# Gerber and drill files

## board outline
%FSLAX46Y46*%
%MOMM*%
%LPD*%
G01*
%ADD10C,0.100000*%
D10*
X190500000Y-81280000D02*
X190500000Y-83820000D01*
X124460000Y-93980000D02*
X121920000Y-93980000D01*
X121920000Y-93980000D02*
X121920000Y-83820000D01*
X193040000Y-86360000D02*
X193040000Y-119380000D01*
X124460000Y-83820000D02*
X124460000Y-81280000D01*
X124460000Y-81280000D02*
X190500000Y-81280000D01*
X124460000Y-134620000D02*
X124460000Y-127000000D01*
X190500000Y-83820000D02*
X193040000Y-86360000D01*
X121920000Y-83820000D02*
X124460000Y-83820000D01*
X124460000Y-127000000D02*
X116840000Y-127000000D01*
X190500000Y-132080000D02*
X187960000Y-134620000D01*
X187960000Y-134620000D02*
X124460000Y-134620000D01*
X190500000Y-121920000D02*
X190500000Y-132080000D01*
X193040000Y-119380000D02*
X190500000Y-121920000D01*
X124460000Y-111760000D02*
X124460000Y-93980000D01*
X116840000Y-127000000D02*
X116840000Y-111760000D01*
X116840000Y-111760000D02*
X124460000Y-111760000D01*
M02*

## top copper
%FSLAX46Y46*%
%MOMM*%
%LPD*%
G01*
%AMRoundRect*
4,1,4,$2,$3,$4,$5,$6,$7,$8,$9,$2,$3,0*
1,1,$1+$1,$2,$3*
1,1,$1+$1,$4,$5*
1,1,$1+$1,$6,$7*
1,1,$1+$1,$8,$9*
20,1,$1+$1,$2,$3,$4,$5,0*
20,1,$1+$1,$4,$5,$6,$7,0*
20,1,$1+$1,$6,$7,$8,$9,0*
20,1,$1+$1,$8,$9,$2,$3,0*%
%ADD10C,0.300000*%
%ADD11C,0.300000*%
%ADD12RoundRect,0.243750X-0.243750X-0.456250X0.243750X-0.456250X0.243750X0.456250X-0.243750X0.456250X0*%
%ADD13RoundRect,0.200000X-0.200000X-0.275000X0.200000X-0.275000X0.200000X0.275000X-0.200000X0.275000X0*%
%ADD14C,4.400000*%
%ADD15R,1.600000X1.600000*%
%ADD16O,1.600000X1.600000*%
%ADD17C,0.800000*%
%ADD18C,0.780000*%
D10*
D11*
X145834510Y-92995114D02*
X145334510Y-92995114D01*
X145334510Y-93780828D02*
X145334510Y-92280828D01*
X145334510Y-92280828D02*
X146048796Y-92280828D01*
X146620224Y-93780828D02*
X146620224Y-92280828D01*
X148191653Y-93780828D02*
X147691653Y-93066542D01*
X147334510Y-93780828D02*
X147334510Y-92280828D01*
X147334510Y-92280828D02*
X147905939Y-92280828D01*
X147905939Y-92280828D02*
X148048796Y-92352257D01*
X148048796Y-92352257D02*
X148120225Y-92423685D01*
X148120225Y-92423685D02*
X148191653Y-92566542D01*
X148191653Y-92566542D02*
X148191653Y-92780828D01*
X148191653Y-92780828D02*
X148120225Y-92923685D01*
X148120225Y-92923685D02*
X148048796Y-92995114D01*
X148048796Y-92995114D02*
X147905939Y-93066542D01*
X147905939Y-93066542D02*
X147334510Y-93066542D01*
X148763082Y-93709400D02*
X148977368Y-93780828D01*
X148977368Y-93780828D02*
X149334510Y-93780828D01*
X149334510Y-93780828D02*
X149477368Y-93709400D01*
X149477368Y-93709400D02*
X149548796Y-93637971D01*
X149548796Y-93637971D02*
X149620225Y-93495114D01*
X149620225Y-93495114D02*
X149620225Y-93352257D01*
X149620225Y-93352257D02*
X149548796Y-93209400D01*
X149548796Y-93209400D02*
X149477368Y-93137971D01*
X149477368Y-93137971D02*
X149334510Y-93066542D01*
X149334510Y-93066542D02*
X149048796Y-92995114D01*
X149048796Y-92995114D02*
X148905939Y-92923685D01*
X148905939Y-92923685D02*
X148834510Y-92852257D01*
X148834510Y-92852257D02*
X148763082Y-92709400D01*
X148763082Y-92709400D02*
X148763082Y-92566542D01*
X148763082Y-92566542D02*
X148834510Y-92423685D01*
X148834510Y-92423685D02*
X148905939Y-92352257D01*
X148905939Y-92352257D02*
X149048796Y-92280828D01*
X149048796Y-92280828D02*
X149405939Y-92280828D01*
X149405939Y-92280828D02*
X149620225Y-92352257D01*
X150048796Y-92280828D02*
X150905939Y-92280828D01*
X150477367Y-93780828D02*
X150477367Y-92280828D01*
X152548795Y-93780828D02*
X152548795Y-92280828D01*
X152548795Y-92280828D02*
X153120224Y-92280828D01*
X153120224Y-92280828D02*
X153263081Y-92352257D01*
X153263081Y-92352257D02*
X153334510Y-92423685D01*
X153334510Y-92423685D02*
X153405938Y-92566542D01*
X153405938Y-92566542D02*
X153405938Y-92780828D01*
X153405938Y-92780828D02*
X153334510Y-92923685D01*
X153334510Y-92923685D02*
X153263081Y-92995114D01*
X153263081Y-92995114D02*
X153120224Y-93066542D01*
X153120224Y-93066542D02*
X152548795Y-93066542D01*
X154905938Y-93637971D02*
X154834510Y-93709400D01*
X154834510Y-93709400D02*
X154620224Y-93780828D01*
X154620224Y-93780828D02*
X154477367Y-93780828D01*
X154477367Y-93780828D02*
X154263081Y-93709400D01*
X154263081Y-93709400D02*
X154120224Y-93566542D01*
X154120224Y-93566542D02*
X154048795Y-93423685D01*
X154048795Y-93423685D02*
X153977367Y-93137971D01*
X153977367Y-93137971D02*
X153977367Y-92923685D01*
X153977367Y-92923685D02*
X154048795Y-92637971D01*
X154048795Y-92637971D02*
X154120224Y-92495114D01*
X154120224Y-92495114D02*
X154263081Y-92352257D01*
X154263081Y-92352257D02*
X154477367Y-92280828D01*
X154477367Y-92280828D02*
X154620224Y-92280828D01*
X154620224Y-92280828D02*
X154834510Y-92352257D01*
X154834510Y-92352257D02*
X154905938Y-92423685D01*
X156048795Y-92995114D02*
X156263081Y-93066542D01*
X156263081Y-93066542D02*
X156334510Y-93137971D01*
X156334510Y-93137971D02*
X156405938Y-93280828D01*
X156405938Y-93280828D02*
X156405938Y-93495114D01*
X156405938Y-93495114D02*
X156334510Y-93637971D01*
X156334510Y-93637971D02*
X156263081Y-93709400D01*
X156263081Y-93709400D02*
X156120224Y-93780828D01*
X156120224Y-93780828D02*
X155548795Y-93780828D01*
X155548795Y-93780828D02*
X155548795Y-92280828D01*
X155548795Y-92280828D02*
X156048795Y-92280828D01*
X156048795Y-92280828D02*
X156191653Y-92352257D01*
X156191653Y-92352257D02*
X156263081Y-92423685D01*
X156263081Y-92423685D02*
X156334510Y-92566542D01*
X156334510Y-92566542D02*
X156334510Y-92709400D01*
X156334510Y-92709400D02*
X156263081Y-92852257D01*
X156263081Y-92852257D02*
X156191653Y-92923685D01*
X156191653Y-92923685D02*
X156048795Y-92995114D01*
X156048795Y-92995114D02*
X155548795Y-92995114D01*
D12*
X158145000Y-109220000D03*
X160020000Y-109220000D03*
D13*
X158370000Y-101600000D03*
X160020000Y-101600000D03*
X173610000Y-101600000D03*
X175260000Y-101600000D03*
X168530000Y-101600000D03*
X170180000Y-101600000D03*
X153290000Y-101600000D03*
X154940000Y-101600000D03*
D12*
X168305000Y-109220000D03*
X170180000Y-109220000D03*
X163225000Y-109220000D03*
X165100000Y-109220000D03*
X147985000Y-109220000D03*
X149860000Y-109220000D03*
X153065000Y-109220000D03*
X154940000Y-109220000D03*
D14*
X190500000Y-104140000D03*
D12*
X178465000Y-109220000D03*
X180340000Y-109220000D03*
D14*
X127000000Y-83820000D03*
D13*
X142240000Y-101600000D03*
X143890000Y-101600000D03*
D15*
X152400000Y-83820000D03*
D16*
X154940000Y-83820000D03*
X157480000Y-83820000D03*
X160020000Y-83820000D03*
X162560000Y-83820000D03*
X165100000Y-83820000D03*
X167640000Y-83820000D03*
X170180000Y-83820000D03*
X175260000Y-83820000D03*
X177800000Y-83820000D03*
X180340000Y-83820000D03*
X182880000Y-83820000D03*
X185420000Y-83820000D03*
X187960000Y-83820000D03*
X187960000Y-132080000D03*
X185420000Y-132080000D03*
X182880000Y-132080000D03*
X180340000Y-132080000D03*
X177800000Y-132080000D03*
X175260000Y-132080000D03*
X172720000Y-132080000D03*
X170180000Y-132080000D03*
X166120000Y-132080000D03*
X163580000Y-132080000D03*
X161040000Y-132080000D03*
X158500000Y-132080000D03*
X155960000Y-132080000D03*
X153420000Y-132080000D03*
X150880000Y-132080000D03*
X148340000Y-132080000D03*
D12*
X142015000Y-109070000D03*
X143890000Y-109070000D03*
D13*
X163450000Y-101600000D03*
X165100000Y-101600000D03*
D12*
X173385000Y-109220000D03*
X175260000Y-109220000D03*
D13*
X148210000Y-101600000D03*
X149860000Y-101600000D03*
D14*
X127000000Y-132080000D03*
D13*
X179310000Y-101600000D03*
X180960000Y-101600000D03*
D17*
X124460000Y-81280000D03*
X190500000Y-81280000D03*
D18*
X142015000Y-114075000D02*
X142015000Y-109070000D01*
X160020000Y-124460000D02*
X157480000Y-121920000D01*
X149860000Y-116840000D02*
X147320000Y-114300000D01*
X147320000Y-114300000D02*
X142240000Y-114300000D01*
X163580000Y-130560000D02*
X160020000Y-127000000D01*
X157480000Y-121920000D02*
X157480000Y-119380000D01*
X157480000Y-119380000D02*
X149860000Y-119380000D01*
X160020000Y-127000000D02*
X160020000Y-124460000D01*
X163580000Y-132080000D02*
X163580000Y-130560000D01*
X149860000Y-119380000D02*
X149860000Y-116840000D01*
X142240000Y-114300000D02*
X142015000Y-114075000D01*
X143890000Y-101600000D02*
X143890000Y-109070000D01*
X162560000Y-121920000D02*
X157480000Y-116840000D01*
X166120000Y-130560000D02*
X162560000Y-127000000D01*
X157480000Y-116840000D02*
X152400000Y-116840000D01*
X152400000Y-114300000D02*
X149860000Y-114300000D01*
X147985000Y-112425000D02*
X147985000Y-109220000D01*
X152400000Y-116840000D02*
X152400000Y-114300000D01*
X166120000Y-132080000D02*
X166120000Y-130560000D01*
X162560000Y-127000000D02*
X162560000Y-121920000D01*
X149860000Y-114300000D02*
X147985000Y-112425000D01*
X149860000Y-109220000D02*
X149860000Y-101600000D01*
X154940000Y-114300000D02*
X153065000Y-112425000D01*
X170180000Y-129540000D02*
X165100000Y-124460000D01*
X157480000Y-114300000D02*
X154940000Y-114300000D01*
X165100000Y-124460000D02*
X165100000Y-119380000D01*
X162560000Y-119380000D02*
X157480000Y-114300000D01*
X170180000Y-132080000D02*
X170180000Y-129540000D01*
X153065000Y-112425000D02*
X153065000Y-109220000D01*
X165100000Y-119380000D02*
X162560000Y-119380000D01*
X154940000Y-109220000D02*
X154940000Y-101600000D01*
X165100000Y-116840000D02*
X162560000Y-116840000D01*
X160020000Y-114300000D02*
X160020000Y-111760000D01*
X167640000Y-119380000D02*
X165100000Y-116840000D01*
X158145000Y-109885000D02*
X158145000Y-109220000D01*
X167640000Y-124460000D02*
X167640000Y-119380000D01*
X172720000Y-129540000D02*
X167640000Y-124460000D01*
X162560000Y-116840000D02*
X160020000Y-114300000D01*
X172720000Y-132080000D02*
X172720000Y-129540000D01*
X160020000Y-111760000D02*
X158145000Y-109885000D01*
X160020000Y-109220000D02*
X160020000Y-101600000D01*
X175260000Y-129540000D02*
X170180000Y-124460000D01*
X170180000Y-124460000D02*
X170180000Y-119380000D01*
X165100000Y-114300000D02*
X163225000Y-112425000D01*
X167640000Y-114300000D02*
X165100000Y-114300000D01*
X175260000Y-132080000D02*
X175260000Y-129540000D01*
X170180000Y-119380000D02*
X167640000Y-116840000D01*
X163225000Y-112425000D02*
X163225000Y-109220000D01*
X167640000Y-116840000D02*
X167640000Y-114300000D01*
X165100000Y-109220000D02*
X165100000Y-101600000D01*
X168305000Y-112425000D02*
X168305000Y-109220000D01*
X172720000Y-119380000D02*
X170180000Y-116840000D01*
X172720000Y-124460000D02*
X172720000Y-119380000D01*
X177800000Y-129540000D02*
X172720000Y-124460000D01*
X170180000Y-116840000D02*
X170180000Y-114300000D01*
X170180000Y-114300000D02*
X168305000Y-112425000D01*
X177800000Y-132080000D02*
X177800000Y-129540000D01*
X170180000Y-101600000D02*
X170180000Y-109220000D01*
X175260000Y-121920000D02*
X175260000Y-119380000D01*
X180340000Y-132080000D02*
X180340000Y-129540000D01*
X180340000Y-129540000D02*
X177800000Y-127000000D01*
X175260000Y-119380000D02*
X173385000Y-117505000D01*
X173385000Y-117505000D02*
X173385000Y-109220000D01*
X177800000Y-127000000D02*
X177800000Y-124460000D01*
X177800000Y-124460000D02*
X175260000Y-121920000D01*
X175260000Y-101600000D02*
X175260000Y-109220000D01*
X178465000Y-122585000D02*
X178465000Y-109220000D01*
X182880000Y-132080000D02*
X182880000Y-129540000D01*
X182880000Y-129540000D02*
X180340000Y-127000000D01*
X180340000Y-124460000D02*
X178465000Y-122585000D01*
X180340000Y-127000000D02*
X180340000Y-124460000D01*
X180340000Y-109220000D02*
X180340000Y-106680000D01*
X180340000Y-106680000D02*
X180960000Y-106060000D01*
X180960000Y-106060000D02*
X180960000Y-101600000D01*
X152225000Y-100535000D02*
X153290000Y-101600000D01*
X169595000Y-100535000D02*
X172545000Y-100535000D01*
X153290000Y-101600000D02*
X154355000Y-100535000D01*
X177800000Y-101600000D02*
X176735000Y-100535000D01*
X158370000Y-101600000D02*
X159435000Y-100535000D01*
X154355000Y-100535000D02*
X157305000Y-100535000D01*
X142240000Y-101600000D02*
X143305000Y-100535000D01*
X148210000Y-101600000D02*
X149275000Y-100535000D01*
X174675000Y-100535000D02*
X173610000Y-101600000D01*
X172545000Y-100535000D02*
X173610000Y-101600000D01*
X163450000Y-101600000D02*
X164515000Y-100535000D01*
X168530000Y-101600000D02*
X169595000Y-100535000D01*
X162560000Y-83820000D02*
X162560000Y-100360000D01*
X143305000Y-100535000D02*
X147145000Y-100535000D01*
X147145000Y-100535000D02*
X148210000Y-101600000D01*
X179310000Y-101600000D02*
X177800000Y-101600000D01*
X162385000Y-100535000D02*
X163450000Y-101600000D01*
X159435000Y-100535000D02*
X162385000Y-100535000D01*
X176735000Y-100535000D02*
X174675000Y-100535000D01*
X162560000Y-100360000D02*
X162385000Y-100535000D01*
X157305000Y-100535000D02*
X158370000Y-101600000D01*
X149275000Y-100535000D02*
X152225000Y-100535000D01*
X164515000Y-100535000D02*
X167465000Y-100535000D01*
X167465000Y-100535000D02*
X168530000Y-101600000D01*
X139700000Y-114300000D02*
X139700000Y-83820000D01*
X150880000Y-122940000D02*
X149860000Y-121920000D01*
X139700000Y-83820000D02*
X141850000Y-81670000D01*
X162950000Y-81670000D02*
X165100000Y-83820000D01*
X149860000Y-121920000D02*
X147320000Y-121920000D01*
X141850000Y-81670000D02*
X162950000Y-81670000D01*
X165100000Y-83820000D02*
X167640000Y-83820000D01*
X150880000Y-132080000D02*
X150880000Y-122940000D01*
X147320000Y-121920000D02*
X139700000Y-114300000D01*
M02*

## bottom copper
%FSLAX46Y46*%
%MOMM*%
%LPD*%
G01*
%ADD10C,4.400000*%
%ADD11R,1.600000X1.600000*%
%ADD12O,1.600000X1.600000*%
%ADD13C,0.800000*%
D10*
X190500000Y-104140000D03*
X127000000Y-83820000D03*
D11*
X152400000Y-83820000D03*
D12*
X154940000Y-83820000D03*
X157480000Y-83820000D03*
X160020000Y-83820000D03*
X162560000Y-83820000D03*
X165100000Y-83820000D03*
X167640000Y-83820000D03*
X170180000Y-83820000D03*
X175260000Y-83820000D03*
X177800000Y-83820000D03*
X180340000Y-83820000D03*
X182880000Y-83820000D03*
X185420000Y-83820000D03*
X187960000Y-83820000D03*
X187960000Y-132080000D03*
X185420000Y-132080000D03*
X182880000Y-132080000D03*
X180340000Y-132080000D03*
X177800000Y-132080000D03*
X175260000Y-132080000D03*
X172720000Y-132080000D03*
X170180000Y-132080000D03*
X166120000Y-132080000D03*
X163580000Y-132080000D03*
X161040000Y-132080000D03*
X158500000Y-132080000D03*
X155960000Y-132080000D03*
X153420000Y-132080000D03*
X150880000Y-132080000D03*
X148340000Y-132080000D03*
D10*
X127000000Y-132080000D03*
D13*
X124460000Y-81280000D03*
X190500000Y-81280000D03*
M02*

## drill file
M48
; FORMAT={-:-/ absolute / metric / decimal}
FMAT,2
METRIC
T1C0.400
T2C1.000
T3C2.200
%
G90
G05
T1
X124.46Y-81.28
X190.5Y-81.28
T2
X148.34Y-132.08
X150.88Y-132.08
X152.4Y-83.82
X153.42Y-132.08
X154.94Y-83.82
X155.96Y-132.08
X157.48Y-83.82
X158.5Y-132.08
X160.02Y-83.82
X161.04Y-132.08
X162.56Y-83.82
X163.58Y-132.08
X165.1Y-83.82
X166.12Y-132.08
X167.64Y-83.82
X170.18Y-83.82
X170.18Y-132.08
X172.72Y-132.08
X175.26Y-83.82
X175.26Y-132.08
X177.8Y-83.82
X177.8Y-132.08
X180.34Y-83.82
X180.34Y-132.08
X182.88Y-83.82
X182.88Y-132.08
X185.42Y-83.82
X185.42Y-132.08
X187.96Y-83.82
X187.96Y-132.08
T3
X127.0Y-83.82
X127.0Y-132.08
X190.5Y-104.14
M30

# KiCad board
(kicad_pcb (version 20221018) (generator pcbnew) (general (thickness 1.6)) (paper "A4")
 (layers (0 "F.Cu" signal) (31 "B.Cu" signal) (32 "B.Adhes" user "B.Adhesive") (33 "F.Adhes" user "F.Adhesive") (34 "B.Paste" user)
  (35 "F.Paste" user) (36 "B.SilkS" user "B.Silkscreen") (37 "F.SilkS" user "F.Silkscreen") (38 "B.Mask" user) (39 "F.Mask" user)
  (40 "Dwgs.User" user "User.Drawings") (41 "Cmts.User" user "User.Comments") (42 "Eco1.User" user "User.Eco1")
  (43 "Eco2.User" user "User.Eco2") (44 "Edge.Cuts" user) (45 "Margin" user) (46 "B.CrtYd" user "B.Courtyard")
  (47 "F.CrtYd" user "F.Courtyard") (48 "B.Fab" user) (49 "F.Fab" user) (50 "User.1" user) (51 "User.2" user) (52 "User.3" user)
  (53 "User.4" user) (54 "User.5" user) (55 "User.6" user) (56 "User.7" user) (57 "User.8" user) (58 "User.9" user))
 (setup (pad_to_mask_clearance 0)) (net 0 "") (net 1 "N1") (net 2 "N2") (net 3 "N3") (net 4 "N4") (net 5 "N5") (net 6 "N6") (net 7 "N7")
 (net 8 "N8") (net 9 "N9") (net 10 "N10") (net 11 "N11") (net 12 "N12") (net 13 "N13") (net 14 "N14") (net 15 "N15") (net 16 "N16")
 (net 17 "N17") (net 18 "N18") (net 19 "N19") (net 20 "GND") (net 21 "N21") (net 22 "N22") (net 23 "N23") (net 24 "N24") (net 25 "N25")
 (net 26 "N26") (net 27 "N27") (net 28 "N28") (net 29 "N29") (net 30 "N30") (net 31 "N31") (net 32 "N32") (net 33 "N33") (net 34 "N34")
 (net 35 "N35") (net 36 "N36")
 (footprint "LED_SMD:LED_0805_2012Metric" (layer "F.Cu") (at 159.0825 109.22)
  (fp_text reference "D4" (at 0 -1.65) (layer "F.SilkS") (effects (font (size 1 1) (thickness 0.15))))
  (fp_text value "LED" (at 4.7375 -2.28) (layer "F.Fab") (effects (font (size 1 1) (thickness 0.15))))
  (pad "1" smd roundrect (at -0.9375 0) (size 0.975 1.4) (layers "F.Cu" "F.Paste" "F.Mask") (roundrect_rratio 0.25) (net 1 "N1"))
  (pad "2" smd roundrect (at 0.9375 0) (size 0.975 1.4) (layers "F.Cu" "F.Paste" "F.Mask") (roundrect_rratio 0.25) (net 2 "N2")))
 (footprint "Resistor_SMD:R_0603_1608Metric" (layer "F.Cu") (at 159.195 101.6)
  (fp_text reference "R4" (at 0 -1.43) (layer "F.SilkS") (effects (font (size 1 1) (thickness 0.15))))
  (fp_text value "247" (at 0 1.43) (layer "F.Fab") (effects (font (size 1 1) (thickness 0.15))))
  (pad "1" smd roundrect (at -0.825 0) (size 0.8 0.95) (layers "F.Cu" "F.Paste" "F.Mask") (roundrect_rratio 0.25) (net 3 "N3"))
  (pad "2" smd roundrect (at 0.825 0) (size 0.8 0.95) (layers "F.Cu" "F.Paste" "F.Mask") (roundrect_rratio 0.25) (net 2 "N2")))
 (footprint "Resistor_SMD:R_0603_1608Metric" (layer "F.Cu") (at 174.435 101.6)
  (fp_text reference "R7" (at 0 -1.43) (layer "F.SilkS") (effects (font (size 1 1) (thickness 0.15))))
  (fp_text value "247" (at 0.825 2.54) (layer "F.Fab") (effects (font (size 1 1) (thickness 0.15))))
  (pad "1" smd roundrect (at -0.825 0) (size 0.8 0.95) (layers "F.Cu" "F.Paste" "F.Mask") (roundrect_rratio 0.25) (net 3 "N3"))
  (pad "2" smd roundrect (at 0.825 0) (size 0.8 0.95) (layers "F.Cu" "F.Paste" "F.Mask") (roundrect_rratio 0.25) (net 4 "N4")))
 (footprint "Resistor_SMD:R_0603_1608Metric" (layer "F.Cu") (at 169.355 101.6)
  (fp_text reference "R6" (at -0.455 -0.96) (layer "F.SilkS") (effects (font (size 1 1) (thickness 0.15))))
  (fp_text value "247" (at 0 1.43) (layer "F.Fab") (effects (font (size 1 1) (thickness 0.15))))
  (pad "1" smd roundrect (at -0.825 0) (size 0.8 0.95) (layers "F.Cu" "F.Paste" "F.Mask") (roundrect_rratio 0.25) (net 3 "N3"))
  (pad "2" smd roundrect (at 0.825 0) (size 0.8 0.95) (layers "F.Cu" "F.Paste" "F.Mask") (roundrect_rratio 0.25) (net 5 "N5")))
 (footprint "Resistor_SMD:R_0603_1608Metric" (layer "F.Cu") (at 154.115 101.6)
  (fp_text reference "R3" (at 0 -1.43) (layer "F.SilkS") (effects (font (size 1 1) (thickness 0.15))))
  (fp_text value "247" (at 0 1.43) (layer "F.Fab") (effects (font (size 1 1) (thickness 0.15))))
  (pad "1" smd roundrect (at -0.825 0) (size 0.8 0.95) (layers "F.Cu" "F.Paste" "F.Mask") (roundrect_rratio 0.25) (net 3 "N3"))
  (pad "2" smd roundrect (at 0.825 0) (size 0.8 0.95) (layers "F.Cu" "F.Paste" "F.Mask") (roundrect_rratio 0.25) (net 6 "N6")))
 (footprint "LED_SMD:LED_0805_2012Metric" (layer "F.Cu") (at 169.2425 109.22)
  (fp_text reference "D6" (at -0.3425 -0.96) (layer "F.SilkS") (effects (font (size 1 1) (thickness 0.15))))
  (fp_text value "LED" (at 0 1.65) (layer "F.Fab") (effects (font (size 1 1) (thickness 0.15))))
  (pad "1" smd roundrect (at -0.9375 0) (size 0.975 1.4) (layers "F.Cu" "F.Paste" "F.Mask") (roundrect_rratio 0.25) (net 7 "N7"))
  (pad "2" smd roundrect (at 0.9375 0) (size 0.975 1.4) (layers "F.Cu" "F.Paste" "F.Mask") (roundrect_rratio 0.25) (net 5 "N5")))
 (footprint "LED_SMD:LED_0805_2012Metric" (layer "F.Cu") (at 164.1625 109.22)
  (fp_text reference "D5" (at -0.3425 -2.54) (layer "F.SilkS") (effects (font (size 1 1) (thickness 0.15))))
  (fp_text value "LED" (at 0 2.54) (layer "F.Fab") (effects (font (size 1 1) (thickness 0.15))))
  (pad "1" smd roundrect (at -0.9375 0) (size 0.975 1.4) (layers "F.Cu" "F.Paste" "F.Mask") (roundrect_rratio 0.25) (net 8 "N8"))
  (pad "2" smd roundrect (at 0.9375 0) (size 0.975 1.4) (layers "F.Cu" "F.Paste" "F.Mask") (roundrect_rratio 0.25) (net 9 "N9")))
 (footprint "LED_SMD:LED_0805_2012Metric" (layer "F.Cu") (at 148.9225 109.22)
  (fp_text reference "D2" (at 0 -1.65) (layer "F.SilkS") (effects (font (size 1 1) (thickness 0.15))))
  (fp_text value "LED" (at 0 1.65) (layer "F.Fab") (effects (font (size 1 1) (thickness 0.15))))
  (pad "1" smd roundrect (at -0.9375 0) (size 0.975 1.4) (layers "F.Cu" "F.Paste" "F.Mask") (roundrect_rratio 0.25) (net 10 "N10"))
  (pad "2" smd roundrect (at 0.9375 0) (size 0.975 1.4) (layers "F.Cu" "F.Paste" "F.Mask") (roundrect_rratio 0.25) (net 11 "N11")))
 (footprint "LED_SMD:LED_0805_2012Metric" (layer "F.Cu") (at 154.0025 109.22)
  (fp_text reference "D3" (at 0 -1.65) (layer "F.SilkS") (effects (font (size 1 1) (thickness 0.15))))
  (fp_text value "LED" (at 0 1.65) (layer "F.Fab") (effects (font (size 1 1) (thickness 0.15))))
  (pad "1" smd roundrect (at -0.9375 0) (size 0.975 1.4) (layers "F.Cu" "F.Paste" "F.Mask") (roundrect_rratio 0.25) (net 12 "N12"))
  (pad "2" smd roundrect (at 0.9375 0) (size 0.975 1.4) (layers "F.Cu" "F.Paste" "F.Mask") (roundrect_rratio 0.25) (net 6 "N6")))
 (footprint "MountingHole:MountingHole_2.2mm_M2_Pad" (layer "F.Cu") (at 190.5 104.14)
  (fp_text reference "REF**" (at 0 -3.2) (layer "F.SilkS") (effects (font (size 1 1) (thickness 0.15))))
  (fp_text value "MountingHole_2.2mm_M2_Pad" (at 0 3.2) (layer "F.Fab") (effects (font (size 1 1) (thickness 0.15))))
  (pad "1" thru_hole circle (at 0 0) (size 4.4 4.4) (drill 2.2) (layers "*.Cu" "*.Mask")))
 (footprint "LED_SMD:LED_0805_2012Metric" (layer "F.Cu") (at 179.4025 109.22)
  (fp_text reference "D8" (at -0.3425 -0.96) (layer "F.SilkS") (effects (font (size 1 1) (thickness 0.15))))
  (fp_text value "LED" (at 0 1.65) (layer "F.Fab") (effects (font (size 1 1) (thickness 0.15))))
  (pad "1" smd roundrect (at -0.9375 0) (size 0.975 1.4) (layers "F.Cu" "F.Paste" "F.Mask") (roundrect_rratio 0.25) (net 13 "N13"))
  (pad "2" smd roundrect (at 0.9375 0) (size 0.975 1.4) (layers "F.Cu" "F.Paste" "F.Mask") (roundrect_rratio 0.25) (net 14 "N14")))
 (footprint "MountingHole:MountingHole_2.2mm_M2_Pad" (layer "F.Cu") (at 127 83.82)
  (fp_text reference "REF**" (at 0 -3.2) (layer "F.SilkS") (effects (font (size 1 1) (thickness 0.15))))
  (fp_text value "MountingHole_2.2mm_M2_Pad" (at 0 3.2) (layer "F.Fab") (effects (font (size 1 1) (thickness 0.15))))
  (pad "1" thru_hole circle (at 0 0) (size 4.4 4.4) (drill 2.2) (layers "*.Cu" "*.Mask")))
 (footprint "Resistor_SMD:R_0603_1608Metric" (layer "F.Cu") (at 143.065 101.6)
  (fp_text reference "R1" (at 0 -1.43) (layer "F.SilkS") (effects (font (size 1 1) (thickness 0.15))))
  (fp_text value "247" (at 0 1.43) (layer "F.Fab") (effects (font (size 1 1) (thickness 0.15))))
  (pad "1" smd roundrect (at -0.825 0) (size 0.8 0.95) (layers "F.Cu" "F.Paste" "F.Mask") (roundrect_rratio 0.25) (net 3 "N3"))
  (pad "2" smd roundrect (at 0.825 0) (size 0.8 0.95) (layers "F.Cu" "F.Paste" "F.Mask") (roundrect_rratio 0.25) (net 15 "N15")))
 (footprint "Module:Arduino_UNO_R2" (layer "F.Cu") (at 152.4 83.82)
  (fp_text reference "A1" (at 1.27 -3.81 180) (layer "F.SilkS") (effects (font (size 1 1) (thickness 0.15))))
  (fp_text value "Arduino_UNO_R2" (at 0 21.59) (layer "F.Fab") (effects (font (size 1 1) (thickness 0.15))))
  (pad "1" thru_hole rect (at 0 0 90) (size 1.6 1.6) (drill 1) (layers "*.Cu" "*.Mask") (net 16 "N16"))
  (pad "2" thru_hole oval (at 2.54 0 90) (size 1.6 1.6) (drill 1) (layers "*.Cu" "*.Mask") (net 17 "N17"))
  (pad "3" thru_hole oval (at 5.08 0 90) (size 1.6 1.6) (drill 1) (layers "*.Cu" "*.Mask") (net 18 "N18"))
  (pad "4" thru_hole oval (at 7.62 0 90) (size 1.6 1.6) (drill 1) (layers "*.Cu" "*.Mask") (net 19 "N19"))
  (pad "5" thru_hole oval (at 10.16 0 90) (size 1.6 1.6) (drill 1) (layers "*.Cu" "*.Mask") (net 3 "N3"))
  (pad "6" thru_hole oval (at 12.7 0 90) (size 1.6 1.6) (drill 1) (layers "*.Cu" "*.Mask") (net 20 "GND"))
  (pad "7" thru_hole oval (at 15.24 0 90) (size 1.6 1.6) (drill 1) (layers "*.Cu" "*.Mask") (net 20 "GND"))
  (pad "8" thru_hole oval (at 17.78 0 90) (size 1.6 1.6) (drill 1) (layers "*.Cu" "*.Mask") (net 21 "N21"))
  (pad "9" thru_hole oval (at 22.86 0 90) (size 1.6 1.6) (drill 1) (layers "*.Cu" "*.Mask") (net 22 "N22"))
  (pad "10" thru_hole oval (at 25.4 0 90) (size 1.6 1.6) (drill 1) (layers "*.Cu" "*.Mask") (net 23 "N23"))
  (pad "11" thru_hole oval (at 27.94 0 90) (size 1.6 1.6) (drill 1) (layers "*.Cu" "*.Mask") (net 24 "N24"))
  (pad "12" thru_hole oval (at 30.48 0 90) (size 1.6 1.6) (drill 1) (layers "*.Cu" "*.Mask") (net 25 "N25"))
  (pad "13" thru_hole oval (at 33.02 0 90) (size 1.6 1.6) (drill 1) (layers "*.Cu" "*.Mask") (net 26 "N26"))
  (pad "14" thru_hole oval (at 35.56 0 90) (size 1.6 1.6) (drill 1) (layers "*.Cu" "*.Mask") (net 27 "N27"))
  (pad "15" thru_hole oval (at 35.56 48.26 90) (size 1.6 1.6) (drill 1) (layers "*.Cu" "*.Mask") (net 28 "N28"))
  (pad "16" thru_hole oval (at 33.02 48.26 90) (size 1.6 1.6) (drill 1) (layers "*.Cu" "*.Mask") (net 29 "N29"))
  (pad "17" thru_hole oval (at 30.48 48.26 90) (size 1.6 1.6) (drill 1) (layers "*.Cu" "*.Mask") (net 13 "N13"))
  (pad "18" thru_hole oval (at 27.94 48.26 90) (size 1.6 1.6) (drill 1) (layers "*.Cu" "*.Mask") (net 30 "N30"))
  (pad "19" thru_hole oval (at 25.4 48.26 90) (size 1.6 1.6) (drill 1) (layers "*.Cu" "*.Mask") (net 7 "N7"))
  (pad "20" thru_hole oval (at 22.86 48.26 90) (size 1.6 1.6) (drill 1) (layers "*.Cu" "*.Mask") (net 8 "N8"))
  (pad "21" thru_hole oval (at 20.32 48.26 90) (size 1.6 1.6) (drill 1) (layers "*.Cu" "*.Mask") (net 1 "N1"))
  (pad "22" thru_hole oval (at 17.78 48.26 90) (size 1.6 1.6) (drill 1) (layers "*.Cu" "*.Mask") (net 12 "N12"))
  (pad "23" thru_hole oval (at 13.72 48.26 90) (size 1.6 1.6) (drill 1) (layers "*.Cu" "*.Mask") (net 10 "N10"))
  (pad "24" thru_hole oval (at 11.18 48.26 90) (size 1.6 1.6) (drill 1) (layers "*.Cu" "*.Mask") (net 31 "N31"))
  (pad "25" thru_hole oval (at 8.64 48.26 90) (size 1.6 1.6) (drill 1) (layers "*.Cu" "*.Mask") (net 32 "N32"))
  (pad "26" thru_hole oval (at 6.1 48.26 90) (size 1.6 1.6) (drill 1) (layers "*.Cu" "*.Mask") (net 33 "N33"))
  (pad "27" thru_hole oval (at 3.56 48.26 90) (size 1.6 1.6) (drill 1) (layers "*.Cu" "*.Mask") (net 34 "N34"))
  (pad "28" thru_hole oval (at 1.02 48.26 90) (size 1.6 1.6) (drill 1) (layers "*.Cu" "*.Mask") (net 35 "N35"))
  (pad "29" thru_hole oval (at -1.52 48.26 90) (size 1.6 1.6) (drill 1) (layers "*.Cu" "*.Mask") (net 20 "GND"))
  (pad "30" thru_hole oval (at -4.06 48.26 90) (size 1.6 1.6) (drill 1) (layers "*.Cu" "*.Mask") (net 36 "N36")))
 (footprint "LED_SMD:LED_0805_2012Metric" (layer "F.Cu") (at 142.9525 109.07)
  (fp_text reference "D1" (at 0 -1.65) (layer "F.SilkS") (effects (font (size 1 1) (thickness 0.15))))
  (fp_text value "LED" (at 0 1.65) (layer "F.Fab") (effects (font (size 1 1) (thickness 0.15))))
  (pad "1" smd roundrect (at -0.9375 0) (size 0.975 1.4) (layers "F.Cu" "F.Paste" "F.Mask") (roundrect_rratio 0.25) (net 31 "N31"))
  (pad "2" smd roundrect (at 0.9375 0) (size 0.975 1.4) (layers "F.Cu" "F.Paste" "F.Mask") (roundrect_rratio 0.25) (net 15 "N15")))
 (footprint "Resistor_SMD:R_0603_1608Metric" (layer "F.Cu") (at 164.275 101.6)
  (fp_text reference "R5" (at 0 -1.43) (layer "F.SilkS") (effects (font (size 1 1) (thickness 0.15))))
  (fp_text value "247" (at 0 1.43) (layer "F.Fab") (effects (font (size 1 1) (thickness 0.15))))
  (pad "1" smd roundrect (at -0.825 0) (size 0.8 0.95) (layers "F.Cu" "F.Paste" "F.Mask") (roundrect_rratio 0.25) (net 3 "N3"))
  (pad "2" smd roundrect (at 0.825 0) (size 0.8 0.95) (layers "F.Cu" "F.Paste" "F.Mask") (roundrect_rratio 0.25) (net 9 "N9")))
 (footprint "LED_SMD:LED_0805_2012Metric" (layer "F.Cu") (at 174.3225 109.22)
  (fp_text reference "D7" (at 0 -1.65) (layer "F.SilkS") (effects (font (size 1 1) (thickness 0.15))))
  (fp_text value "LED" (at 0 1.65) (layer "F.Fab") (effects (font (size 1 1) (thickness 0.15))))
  (pad "1" smd roundrect (at -0.9375 0) (size 0.975 1.4) (layers "F.Cu" "F.Paste" "F.Mask") (roundrect_rratio 0.25) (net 30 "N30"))
  (pad "2" smd roundrect (at 0.9375 0) (size 0.975 1.4) (layers "F.Cu" "F.Paste" "F.Mask") (roundrect_rratio 0.25) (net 4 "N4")))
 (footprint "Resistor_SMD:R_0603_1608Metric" (layer "F.Cu") (at 149.035 101.6)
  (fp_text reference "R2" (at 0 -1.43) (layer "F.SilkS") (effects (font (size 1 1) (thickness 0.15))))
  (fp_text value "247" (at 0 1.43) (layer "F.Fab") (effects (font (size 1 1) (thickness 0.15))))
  (pad "1" smd roundrect (at -0.825 0) (size 0.8 0.95) (layers "F.Cu" "F.Paste" "F.Mask") (roundrect_rratio 0.25) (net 3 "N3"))
  (pad "2" smd roundrect (at 0.825 0) (size 0.8 0.95) (layers "F.Cu" "F.Paste" "F.Mask") (roundrect_rratio 0.25) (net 11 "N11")))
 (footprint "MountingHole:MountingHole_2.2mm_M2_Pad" (layer "F.Cu") (at 127 132.08)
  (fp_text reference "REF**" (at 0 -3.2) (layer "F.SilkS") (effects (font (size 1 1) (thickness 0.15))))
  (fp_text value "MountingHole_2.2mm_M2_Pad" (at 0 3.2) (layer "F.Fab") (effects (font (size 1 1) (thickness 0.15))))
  (pad "1" thru_hole circle (at 0 0) (size 4.4 4.4) (drill 2.2) (layers "*.Cu" "*.Mask")))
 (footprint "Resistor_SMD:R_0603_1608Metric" (layer "F.Cu") (at 180.135 101.6)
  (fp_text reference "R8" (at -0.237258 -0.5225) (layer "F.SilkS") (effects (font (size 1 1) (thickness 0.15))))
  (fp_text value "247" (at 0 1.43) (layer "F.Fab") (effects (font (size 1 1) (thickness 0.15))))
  (pad "1" smd roundrect (at -0.825 0) (size 0.8 0.95) (layers "F.Cu" "F.Paste" "F.Mask") (roundrect_rratio 0.25) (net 3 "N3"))
  (pad "2" smd roundrect (at 0.825 0) (size 0.8 0.95) (layers "F.Cu" "F.Paste" "F.Mask") (roundrect_rratio 0.25) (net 14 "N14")))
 (gr_line (start 190.5 81.28) (end 190.5 83.82) (stroke (width 0.1) (type default)) (layer "Edge.Cuts"))
 (gr_line (start 124.46 93.98) (end 121.92 93.98) (stroke (width 0.1) (type default)) (layer "Edge.Cuts"))
 (gr_line (start 121.92 93.98) (end 121.92 83.82) (stroke (width 0.1) (type default)) (layer "Edge.Cuts"))
 (gr_line (start 193.04 86.36) (end 193.04 119.38) (stroke (width 0.1) (type default)) (layer "Edge.Cuts"))
 (gr_line (start 124.46 83.82) (end 124.46 81.28) (stroke (width 0.1) (type default)) (layer "Edge.Cuts"))
 (gr_line (start 124.46 81.28) (end 190.5 81.28) (stroke (width 0.1) (type default)) (layer "Edge.Cuts"))
 (gr_line (start 124.46 134.62) (end 124.46 127) (stroke (width 0.1) (type default)) (layer "Edge.Cuts"))
 (gr_line (start 190.5 83.82) (end 193.04 86.36) (stroke (width 0.1) (type default)) (layer "Edge.Cuts"))
 (gr_line (start 121.92 83.82) (end 124.46 83.82) (stroke (width 0.1) (type default)) (layer "Edge.Cuts"))
 (gr_line (start 124.46 127) (end 116.84 127) (stroke (width 0.1) (type default)) (layer "Edge.Cuts"))
 (gr_line (start 190.5 132.08) (end 187.96 134.62) (stroke (width 0.1) (type default)) (layer "Edge.Cuts"))
 (gr_line (start 187.96 134.62) (end 124.46 134.62) (stroke (width 0.1) (type default)) (layer "Edge.Cuts"))
 (gr_line (start 190.5 121.92) (end 190.5 132.08) (stroke (width 0.1) (type default)) (layer "Edge.Cuts"))
 (gr_line (start 193.04 119.38) (end 190.5 121.92) (stroke (width 0.1) (type default)) (layer "Edge.Cuts"))
 (gr_line (start 124.46 111.76) (end 124.46 93.98) (stroke (width 0.1) (type default)) (layer "Edge.Cuts"))
 (gr_line (start 116.84 127) (end 116.84 111.76) (stroke (width 0.1) (type default)) (layer "Edge.Cuts"))
 (gr_line (start 116.84 111.76) (end 124.46 111.76) (stroke (width 0.1) (type default)) (layer "Edge.Cuts"))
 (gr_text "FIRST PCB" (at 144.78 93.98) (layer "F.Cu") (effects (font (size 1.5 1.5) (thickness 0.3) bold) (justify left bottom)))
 (via (at 124.46 81.28) (size 0.8) (drill 0.4) (layers "F.Cu" "B.Cu") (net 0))
 (via (at 190.5 81.28) (size 0.8) (drill 0.4) (layers "F.Cu" "B.Cu") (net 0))
 (segment (start 142.015 114.075) (end 142.015 109.07) (width 0.78) (layer "F.Cu") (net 31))
 (segment (start 160.02 124.46) (end 157.48 121.92) (width 0.78) (layer "F.Cu") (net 31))
 (segment (start 149.86 116.84) (end 147.32 114.3) (width 0.78) (layer "F.Cu") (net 31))
 (segment (start 147.32 114.3) (end 142.24 114.3) (width 0.78) (layer "F.Cu") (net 31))
 (segment (start 163.58 130.56) (end 160.02 127) (width 0.78) (layer "F.Cu") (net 31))
 (segment (start 157.48 121.92) (end 157.48 119.38) (width 0.78) (layer "F.Cu") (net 31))
 (segment (start 157.48 119.38) (end 149.86 119.38) (width 0.78) (layer "F.Cu") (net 31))
 (segment (start 160.02 127) (end 160.02 124.46) (width 0.78) (layer "F.Cu") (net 31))
 (segment (start 163.58 132.08) (end 163.58 130.56) (width 0.78) (layer "F.Cu") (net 31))
 (segment (start 149.86 119.38) (end 149.86 116.84) (width 0.78) (layer "F.Cu") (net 31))
 (segment (start 142.24 114.3) (end 142.015 114.075) (width 0.78) (layer "F.Cu") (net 31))
 (segment (start 143.89 101.6) (end 143.89 109.07) (width 0.78) (layer "F.Cu") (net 15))
 (segment (start 162.56 121.92) (end 157.48 116.84) (width 0.78) (layer "F.Cu") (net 10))
 (segment (start 166.12 130.56) (end 162.56 127) (width 0.78) (layer "F.Cu") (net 10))
 (segment (start 157.48 116.84) (end 152.4 116.84) (width 0.78) (layer "F.Cu") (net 10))
 (segment (start 152.4 114.3) (end 149.86 114.3) (width 0.78) (layer "F.Cu") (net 10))
 (segment (start 147.985 112.425) (end 147.985 109.22) (width 0.78) (layer "F.Cu") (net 10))
 (segment (start 152.4 116.84) (end 152.4 114.3) (width 0.78) (layer "F.Cu") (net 10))
 (segment (start 166.12 132.08) (end 166.12 130.56) (width 0.78) (layer "F.Cu") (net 10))
 (segment (start 162.56 127) (end 162.56 121.92) (width 0.78) (layer "F.Cu") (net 10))
 (segment (start 149.86 114.3) (end 147.985 112.425) (width 0.78) (layer "F.Cu") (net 10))
 (segment (start 149.86 109.22) (end 149.86 101.6) (width 0.78) (layer "F.Cu") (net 11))
 (segment (start 154.94 114.3) (end 153.065 112.425) (width 0.78) (layer "F.Cu") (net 12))
 (segment (start 170.18 129.54) (end 165.1 124.46) (width 0.78) (layer "F.Cu") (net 12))
 (segment (start 157.48 114.3) (end 154.94 114.3) (width 0.78) (layer "F.Cu") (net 12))
 (segment (start 165.1 124.46) (end 165.1 119.38) (width 0.78) (layer "F.Cu") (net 12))
 (segment (start 162.56 119.38) (end 157.48 114.3) (width 0.78) (layer "F.Cu") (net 12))
 (segment (start 170.18 132.08) (end 170.18 129.54) (width 0.78) (layer "F.Cu") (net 12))
 (segment (start 153.065 112.425) (end 153.065 109.22) (width 0.78) (layer "F.Cu") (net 12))
 (segment (start 165.1 119.38) (end 162.56 119.38) (width 0.78) (layer "F.Cu") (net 12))
 (segment (start 154.94 109.22) (end 154.94 101.6) (width 0.78) (layer "F.Cu") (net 6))
 (segment (start 165.1 116.84) (end 162.56 116.84) (width 0.78) (layer "F.Cu") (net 1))
 (segment (start 160.02 114.3) (end 160.02 111.76) (width 0.78) (layer "F.Cu") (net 1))
 (segment (start 167.64 119.38) (end 165.1 116.84) (width 0.78) (layer "F.Cu") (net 1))
 (segment (start 158.145 109.885) (end 158.145 109.22) (width 0.78) (layer "F.Cu") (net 1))
 (segment (start 167.64 124.46) (end 167.64 119.38) (width 0.78) (layer "F.Cu") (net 1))
 (segment (start 172.72 129.54) (end 167.64 124.46) (width 0.78) (layer "F.Cu") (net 1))
 (segment (start 162.56 116.84) (end 160.02 114.3) (width 0.78) (layer "F.Cu") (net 1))
 (segment (start 172.72 132.08) (end 172.72 129.54) (width 0.78) (layer "F.Cu") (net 1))
 (segment (start 160.02 111.76) (end 158.145 109.885) (width 0.78) (layer "F.Cu") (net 1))
 (segment (start 160.02 109.22) (end 160.02 101.6) (width 0.78) (layer "F.Cu") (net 2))
 (segment (start 175.26 129.54) (end 170.18 124.46) (width 0.78) (layer "F.Cu") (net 8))
 (segment (start 170.18 124.46) (end 170.18 119.38) (width 0.78) (layer "F.Cu") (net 8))
 (segment (start 165.1 114.3) (end 163.225 112.425) (width 0.78) (layer "F.Cu") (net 8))
 (segment (start 167.64 114.3) (end 165.1 114.3) (width 0.78) (layer "F.Cu") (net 8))
 (segment (start 175.26 132.08) (end 175.26 129.54) (width 0.78) (layer "F.Cu") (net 8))
 (segment (start 170.18 119.38) (end 167.64 116.84) (width 0.78) (layer "F.Cu") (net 8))
 (segment (start 163.225 112.425) (end 163.225 109.22) (width 0.78) (layer "F.Cu") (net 8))
 (segment (start 167.64 116.84) (end 167.64 114.3) (width 0.78) (layer "F.Cu") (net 8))
 (segment (start 165.1 109.22) (end 165.1 101.6) (width 0.78) (layer "F.Cu") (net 9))
 (segment (start 168.305 112.425) (end 168.305 109.22) (width 0.78) (layer "F.Cu") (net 7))
 (segment (start 172.72 119.38) (end 170.18 116.84) (width 0.78) (layer "F.Cu") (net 7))
 (segment (start 172.72 124.46) (end 172.72 119.38) (width 0.78) (layer "F.Cu") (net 7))
 (segment (start 177.8 129.54) (end 172.72 124.46) (width 0.78) (layer "F.Cu") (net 7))
 (segment (start 170.18 116.84) (end 170.18 114.3) (width 0.78) (layer "F.Cu") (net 7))
 (segment (start 170.18 114.3) (end 168.305 112.425) (width 0.78) (layer "F.Cu") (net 7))
 (segment (start 177.8 132.08) (end 177.8 129.54) (width 0.78) (layer "F.Cu") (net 7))
 (segment (start 170.18 101.6) (end 170.18 109.22) (width 0.78) (layer "F.Cu") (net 5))
 (segment (start 175.26 121.92) (end 175.26 119.38) (width 0.78) (layer "F.Cu") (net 30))
 (segment (start 180.34 132.08) (end 180.34 129.54) (width 0.78) (layer "F.Cu") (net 30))
 (segment (start 180.34 129.54) (end 177.8 127) (width 0.78) (layer "F.Cu") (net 30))
 (segment (start 175.26 119.38) (end 173.385 117.505) (width 0.78) (layer "F.Cu") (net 30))
 (segment (start 173.385 117.505) (end 173.385 109.22) (width 0.78) (layer "F.Cu") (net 30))
 (segment (start 177.8 127) (end 177.8 124.46) (width 0.78) (layer "F.Cu") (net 30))
 (segment (start 177.8 124.46) (end 175.26 121.92) (width 0.78) (layer "F.Cu") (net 30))
 (segment (start 175.26 101.6) (end 175.26 109.22) (width 0.78) (layer "F.Cu") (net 4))
 (segment (start 178.465 122.585) (end 178.465 109.22) (width 0.78) (layer "F.Cu") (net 13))
 (segment (start 182.88 132.08) (end 182.88 129.54) (width 0.78) (layer "F.Cu") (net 13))
 (segment (start 182.88 129.54) (end 180.34 127) (width 0.78) (layer "F.Cu") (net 13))
 (segment (start 180.34 124.46) (end 178.465 122.585) (width 0.78) (layer "F.Cu") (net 13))
 (segment (start 180.34 127) (end 180.34 124.46) (width 0.78) (layer "F.Cu") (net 13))
 (segment (start 180.34 109.22) (end 180.34 106.68) (width 0.78) (layer "F.Cu") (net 14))
 (segment (start 180.34 106.68) (end 180.96 106.06) (width 0.78) (layer "F.Cu") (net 14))
 (segment (start 180.96 106.06) (end 180.96 101.6) (width 0.78) (layer "F.Cu") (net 14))
 (segment (start 152.225 100.535) (end 153.29 101.6) (width 0.78) (layer "F.Cu") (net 3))
 (segment (start 169.595 100.535) (end 172.545 100.535) (width 0.78) (layer "F.Cu") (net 3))
 (segment (start 153.29 101.6) (end 154.355 100.535) (width 0.78) (layer "F.Cu") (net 3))
 (segment (start 177.8 101.6) (end 176.735 100.535) (width 0.78) (layer "F.Cu") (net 3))
 (segment (start 158.37 101.6) (end 159.435 100.535) (width 0.78) (layer "F.Cu") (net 3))
 (segment (start 154.355 100.535) (end 157.305 100.535) (width 0.78) (layer "F.Cu") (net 3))
 (segment (start 142.24 101.6) (end 143.305 100.535) (width 0.78) (layer "F.Cu") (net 3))
 (segment (start 148.21 101.6) (end 149.275 100.535) (width 0.78) (layer "F.Cu") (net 3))
 (segment (start 174.675 100.535) (end 173.61 101.6) (width 0.78) (layer "F.Cu") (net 3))
 (segment (start 172.545 100.535) (end 173.61 101.6) (width 0.78) (layer "F.Cu") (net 3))
 (segment (start 163.45 101.6) (end 164.515 100.535) (width 0.78) (layer "F.Cu") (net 3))
 (segment (start 168.53 101.6) (end 169.595 100.535) (width 0.78) (layer "F.Cu") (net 3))
 (segment (start 162.56 83.82) (end 162.56 100.36) (width 0.78) (layer "F.Cu") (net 3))
 (segment (start 143.305 100.535) (end 147.145 100.535) (width 0.78) (layer "F.Cu") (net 3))
 (segment (start 147.145 100.535) (end 148.21 101.6) (width 0.78) (layer "F.Cu") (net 3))
 (segment (start 179.31 101.6) (end 177.8 101.6) (width 0.78) (layer "F.Cu") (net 3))
 (segment (start 162.385 100.535) (end 163.45 101.6) (width 0.78) (layer "F.Cu") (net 3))
 (segment (start 159.435 100.535) (end 162.385 100.535) (width 0.78) (layer "F.Cu") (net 3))
 (segment (start 176.735 100.535) (end 174.675 100.535) (width 0.78) (layer "F.Cu") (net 3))
 (segment (start 162.56 100.36) (end 162.385 100.535) (width 0.78) (layer "F.Cu") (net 3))
 (segment (start 157.305 100.535) (end 158.37 101.6) (width 0.78) (layer "F.Cu") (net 3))
 (segment (start 149.275 100.535) (end 152.225 100.535) (width 0.78) (layer "F.Cu") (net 3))
 (segment (start 164.515 100.535) (end 167.465 100.535) (width 0.78) (layer "F.Cu") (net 3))
 (segment (start 167.465 100.535) (end 168.53 101.6) (width 0.78) (layer "F.Cu") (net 3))
 (segment (start 139.7 114.3) (end 139.7 83.82) (width 0.78) (layer "F.Cu") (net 20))
 (segment (start 150.88 122.94) (end 149.86 121.92) (width 0.78) (layer "F.Cu") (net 20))
 (segment (start 139.7 83.82) (end 141.85 81.67) (width 0.78) (layer "F.Cu") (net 20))
 (segment (start 162.95 81.67) (end 165.1 83.82) (width 0.78) (layer "F.Cu") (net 20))
 (segment (start 149.86 121.92) (end 147.32 121.92) (width 0.78) (layer "F.Cu") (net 20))
 (segment (start 141.85 81.67) (end 162.95 81.67) (width 0.78) (layer "F.Cu") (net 20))
 (segment (start 165.1 83.82) (end 167.64 83.82) (width 0.78) (layer "F.Cu") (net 20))
 (segment (start 150.88 132.08) (end 150.88 122.94) (width 0.78) (layer "F.Cu") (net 20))
 (segment (start 147.32 121.92) (end 139.7 114.3) (width 0.78) (layer "F.Cu") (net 20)))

